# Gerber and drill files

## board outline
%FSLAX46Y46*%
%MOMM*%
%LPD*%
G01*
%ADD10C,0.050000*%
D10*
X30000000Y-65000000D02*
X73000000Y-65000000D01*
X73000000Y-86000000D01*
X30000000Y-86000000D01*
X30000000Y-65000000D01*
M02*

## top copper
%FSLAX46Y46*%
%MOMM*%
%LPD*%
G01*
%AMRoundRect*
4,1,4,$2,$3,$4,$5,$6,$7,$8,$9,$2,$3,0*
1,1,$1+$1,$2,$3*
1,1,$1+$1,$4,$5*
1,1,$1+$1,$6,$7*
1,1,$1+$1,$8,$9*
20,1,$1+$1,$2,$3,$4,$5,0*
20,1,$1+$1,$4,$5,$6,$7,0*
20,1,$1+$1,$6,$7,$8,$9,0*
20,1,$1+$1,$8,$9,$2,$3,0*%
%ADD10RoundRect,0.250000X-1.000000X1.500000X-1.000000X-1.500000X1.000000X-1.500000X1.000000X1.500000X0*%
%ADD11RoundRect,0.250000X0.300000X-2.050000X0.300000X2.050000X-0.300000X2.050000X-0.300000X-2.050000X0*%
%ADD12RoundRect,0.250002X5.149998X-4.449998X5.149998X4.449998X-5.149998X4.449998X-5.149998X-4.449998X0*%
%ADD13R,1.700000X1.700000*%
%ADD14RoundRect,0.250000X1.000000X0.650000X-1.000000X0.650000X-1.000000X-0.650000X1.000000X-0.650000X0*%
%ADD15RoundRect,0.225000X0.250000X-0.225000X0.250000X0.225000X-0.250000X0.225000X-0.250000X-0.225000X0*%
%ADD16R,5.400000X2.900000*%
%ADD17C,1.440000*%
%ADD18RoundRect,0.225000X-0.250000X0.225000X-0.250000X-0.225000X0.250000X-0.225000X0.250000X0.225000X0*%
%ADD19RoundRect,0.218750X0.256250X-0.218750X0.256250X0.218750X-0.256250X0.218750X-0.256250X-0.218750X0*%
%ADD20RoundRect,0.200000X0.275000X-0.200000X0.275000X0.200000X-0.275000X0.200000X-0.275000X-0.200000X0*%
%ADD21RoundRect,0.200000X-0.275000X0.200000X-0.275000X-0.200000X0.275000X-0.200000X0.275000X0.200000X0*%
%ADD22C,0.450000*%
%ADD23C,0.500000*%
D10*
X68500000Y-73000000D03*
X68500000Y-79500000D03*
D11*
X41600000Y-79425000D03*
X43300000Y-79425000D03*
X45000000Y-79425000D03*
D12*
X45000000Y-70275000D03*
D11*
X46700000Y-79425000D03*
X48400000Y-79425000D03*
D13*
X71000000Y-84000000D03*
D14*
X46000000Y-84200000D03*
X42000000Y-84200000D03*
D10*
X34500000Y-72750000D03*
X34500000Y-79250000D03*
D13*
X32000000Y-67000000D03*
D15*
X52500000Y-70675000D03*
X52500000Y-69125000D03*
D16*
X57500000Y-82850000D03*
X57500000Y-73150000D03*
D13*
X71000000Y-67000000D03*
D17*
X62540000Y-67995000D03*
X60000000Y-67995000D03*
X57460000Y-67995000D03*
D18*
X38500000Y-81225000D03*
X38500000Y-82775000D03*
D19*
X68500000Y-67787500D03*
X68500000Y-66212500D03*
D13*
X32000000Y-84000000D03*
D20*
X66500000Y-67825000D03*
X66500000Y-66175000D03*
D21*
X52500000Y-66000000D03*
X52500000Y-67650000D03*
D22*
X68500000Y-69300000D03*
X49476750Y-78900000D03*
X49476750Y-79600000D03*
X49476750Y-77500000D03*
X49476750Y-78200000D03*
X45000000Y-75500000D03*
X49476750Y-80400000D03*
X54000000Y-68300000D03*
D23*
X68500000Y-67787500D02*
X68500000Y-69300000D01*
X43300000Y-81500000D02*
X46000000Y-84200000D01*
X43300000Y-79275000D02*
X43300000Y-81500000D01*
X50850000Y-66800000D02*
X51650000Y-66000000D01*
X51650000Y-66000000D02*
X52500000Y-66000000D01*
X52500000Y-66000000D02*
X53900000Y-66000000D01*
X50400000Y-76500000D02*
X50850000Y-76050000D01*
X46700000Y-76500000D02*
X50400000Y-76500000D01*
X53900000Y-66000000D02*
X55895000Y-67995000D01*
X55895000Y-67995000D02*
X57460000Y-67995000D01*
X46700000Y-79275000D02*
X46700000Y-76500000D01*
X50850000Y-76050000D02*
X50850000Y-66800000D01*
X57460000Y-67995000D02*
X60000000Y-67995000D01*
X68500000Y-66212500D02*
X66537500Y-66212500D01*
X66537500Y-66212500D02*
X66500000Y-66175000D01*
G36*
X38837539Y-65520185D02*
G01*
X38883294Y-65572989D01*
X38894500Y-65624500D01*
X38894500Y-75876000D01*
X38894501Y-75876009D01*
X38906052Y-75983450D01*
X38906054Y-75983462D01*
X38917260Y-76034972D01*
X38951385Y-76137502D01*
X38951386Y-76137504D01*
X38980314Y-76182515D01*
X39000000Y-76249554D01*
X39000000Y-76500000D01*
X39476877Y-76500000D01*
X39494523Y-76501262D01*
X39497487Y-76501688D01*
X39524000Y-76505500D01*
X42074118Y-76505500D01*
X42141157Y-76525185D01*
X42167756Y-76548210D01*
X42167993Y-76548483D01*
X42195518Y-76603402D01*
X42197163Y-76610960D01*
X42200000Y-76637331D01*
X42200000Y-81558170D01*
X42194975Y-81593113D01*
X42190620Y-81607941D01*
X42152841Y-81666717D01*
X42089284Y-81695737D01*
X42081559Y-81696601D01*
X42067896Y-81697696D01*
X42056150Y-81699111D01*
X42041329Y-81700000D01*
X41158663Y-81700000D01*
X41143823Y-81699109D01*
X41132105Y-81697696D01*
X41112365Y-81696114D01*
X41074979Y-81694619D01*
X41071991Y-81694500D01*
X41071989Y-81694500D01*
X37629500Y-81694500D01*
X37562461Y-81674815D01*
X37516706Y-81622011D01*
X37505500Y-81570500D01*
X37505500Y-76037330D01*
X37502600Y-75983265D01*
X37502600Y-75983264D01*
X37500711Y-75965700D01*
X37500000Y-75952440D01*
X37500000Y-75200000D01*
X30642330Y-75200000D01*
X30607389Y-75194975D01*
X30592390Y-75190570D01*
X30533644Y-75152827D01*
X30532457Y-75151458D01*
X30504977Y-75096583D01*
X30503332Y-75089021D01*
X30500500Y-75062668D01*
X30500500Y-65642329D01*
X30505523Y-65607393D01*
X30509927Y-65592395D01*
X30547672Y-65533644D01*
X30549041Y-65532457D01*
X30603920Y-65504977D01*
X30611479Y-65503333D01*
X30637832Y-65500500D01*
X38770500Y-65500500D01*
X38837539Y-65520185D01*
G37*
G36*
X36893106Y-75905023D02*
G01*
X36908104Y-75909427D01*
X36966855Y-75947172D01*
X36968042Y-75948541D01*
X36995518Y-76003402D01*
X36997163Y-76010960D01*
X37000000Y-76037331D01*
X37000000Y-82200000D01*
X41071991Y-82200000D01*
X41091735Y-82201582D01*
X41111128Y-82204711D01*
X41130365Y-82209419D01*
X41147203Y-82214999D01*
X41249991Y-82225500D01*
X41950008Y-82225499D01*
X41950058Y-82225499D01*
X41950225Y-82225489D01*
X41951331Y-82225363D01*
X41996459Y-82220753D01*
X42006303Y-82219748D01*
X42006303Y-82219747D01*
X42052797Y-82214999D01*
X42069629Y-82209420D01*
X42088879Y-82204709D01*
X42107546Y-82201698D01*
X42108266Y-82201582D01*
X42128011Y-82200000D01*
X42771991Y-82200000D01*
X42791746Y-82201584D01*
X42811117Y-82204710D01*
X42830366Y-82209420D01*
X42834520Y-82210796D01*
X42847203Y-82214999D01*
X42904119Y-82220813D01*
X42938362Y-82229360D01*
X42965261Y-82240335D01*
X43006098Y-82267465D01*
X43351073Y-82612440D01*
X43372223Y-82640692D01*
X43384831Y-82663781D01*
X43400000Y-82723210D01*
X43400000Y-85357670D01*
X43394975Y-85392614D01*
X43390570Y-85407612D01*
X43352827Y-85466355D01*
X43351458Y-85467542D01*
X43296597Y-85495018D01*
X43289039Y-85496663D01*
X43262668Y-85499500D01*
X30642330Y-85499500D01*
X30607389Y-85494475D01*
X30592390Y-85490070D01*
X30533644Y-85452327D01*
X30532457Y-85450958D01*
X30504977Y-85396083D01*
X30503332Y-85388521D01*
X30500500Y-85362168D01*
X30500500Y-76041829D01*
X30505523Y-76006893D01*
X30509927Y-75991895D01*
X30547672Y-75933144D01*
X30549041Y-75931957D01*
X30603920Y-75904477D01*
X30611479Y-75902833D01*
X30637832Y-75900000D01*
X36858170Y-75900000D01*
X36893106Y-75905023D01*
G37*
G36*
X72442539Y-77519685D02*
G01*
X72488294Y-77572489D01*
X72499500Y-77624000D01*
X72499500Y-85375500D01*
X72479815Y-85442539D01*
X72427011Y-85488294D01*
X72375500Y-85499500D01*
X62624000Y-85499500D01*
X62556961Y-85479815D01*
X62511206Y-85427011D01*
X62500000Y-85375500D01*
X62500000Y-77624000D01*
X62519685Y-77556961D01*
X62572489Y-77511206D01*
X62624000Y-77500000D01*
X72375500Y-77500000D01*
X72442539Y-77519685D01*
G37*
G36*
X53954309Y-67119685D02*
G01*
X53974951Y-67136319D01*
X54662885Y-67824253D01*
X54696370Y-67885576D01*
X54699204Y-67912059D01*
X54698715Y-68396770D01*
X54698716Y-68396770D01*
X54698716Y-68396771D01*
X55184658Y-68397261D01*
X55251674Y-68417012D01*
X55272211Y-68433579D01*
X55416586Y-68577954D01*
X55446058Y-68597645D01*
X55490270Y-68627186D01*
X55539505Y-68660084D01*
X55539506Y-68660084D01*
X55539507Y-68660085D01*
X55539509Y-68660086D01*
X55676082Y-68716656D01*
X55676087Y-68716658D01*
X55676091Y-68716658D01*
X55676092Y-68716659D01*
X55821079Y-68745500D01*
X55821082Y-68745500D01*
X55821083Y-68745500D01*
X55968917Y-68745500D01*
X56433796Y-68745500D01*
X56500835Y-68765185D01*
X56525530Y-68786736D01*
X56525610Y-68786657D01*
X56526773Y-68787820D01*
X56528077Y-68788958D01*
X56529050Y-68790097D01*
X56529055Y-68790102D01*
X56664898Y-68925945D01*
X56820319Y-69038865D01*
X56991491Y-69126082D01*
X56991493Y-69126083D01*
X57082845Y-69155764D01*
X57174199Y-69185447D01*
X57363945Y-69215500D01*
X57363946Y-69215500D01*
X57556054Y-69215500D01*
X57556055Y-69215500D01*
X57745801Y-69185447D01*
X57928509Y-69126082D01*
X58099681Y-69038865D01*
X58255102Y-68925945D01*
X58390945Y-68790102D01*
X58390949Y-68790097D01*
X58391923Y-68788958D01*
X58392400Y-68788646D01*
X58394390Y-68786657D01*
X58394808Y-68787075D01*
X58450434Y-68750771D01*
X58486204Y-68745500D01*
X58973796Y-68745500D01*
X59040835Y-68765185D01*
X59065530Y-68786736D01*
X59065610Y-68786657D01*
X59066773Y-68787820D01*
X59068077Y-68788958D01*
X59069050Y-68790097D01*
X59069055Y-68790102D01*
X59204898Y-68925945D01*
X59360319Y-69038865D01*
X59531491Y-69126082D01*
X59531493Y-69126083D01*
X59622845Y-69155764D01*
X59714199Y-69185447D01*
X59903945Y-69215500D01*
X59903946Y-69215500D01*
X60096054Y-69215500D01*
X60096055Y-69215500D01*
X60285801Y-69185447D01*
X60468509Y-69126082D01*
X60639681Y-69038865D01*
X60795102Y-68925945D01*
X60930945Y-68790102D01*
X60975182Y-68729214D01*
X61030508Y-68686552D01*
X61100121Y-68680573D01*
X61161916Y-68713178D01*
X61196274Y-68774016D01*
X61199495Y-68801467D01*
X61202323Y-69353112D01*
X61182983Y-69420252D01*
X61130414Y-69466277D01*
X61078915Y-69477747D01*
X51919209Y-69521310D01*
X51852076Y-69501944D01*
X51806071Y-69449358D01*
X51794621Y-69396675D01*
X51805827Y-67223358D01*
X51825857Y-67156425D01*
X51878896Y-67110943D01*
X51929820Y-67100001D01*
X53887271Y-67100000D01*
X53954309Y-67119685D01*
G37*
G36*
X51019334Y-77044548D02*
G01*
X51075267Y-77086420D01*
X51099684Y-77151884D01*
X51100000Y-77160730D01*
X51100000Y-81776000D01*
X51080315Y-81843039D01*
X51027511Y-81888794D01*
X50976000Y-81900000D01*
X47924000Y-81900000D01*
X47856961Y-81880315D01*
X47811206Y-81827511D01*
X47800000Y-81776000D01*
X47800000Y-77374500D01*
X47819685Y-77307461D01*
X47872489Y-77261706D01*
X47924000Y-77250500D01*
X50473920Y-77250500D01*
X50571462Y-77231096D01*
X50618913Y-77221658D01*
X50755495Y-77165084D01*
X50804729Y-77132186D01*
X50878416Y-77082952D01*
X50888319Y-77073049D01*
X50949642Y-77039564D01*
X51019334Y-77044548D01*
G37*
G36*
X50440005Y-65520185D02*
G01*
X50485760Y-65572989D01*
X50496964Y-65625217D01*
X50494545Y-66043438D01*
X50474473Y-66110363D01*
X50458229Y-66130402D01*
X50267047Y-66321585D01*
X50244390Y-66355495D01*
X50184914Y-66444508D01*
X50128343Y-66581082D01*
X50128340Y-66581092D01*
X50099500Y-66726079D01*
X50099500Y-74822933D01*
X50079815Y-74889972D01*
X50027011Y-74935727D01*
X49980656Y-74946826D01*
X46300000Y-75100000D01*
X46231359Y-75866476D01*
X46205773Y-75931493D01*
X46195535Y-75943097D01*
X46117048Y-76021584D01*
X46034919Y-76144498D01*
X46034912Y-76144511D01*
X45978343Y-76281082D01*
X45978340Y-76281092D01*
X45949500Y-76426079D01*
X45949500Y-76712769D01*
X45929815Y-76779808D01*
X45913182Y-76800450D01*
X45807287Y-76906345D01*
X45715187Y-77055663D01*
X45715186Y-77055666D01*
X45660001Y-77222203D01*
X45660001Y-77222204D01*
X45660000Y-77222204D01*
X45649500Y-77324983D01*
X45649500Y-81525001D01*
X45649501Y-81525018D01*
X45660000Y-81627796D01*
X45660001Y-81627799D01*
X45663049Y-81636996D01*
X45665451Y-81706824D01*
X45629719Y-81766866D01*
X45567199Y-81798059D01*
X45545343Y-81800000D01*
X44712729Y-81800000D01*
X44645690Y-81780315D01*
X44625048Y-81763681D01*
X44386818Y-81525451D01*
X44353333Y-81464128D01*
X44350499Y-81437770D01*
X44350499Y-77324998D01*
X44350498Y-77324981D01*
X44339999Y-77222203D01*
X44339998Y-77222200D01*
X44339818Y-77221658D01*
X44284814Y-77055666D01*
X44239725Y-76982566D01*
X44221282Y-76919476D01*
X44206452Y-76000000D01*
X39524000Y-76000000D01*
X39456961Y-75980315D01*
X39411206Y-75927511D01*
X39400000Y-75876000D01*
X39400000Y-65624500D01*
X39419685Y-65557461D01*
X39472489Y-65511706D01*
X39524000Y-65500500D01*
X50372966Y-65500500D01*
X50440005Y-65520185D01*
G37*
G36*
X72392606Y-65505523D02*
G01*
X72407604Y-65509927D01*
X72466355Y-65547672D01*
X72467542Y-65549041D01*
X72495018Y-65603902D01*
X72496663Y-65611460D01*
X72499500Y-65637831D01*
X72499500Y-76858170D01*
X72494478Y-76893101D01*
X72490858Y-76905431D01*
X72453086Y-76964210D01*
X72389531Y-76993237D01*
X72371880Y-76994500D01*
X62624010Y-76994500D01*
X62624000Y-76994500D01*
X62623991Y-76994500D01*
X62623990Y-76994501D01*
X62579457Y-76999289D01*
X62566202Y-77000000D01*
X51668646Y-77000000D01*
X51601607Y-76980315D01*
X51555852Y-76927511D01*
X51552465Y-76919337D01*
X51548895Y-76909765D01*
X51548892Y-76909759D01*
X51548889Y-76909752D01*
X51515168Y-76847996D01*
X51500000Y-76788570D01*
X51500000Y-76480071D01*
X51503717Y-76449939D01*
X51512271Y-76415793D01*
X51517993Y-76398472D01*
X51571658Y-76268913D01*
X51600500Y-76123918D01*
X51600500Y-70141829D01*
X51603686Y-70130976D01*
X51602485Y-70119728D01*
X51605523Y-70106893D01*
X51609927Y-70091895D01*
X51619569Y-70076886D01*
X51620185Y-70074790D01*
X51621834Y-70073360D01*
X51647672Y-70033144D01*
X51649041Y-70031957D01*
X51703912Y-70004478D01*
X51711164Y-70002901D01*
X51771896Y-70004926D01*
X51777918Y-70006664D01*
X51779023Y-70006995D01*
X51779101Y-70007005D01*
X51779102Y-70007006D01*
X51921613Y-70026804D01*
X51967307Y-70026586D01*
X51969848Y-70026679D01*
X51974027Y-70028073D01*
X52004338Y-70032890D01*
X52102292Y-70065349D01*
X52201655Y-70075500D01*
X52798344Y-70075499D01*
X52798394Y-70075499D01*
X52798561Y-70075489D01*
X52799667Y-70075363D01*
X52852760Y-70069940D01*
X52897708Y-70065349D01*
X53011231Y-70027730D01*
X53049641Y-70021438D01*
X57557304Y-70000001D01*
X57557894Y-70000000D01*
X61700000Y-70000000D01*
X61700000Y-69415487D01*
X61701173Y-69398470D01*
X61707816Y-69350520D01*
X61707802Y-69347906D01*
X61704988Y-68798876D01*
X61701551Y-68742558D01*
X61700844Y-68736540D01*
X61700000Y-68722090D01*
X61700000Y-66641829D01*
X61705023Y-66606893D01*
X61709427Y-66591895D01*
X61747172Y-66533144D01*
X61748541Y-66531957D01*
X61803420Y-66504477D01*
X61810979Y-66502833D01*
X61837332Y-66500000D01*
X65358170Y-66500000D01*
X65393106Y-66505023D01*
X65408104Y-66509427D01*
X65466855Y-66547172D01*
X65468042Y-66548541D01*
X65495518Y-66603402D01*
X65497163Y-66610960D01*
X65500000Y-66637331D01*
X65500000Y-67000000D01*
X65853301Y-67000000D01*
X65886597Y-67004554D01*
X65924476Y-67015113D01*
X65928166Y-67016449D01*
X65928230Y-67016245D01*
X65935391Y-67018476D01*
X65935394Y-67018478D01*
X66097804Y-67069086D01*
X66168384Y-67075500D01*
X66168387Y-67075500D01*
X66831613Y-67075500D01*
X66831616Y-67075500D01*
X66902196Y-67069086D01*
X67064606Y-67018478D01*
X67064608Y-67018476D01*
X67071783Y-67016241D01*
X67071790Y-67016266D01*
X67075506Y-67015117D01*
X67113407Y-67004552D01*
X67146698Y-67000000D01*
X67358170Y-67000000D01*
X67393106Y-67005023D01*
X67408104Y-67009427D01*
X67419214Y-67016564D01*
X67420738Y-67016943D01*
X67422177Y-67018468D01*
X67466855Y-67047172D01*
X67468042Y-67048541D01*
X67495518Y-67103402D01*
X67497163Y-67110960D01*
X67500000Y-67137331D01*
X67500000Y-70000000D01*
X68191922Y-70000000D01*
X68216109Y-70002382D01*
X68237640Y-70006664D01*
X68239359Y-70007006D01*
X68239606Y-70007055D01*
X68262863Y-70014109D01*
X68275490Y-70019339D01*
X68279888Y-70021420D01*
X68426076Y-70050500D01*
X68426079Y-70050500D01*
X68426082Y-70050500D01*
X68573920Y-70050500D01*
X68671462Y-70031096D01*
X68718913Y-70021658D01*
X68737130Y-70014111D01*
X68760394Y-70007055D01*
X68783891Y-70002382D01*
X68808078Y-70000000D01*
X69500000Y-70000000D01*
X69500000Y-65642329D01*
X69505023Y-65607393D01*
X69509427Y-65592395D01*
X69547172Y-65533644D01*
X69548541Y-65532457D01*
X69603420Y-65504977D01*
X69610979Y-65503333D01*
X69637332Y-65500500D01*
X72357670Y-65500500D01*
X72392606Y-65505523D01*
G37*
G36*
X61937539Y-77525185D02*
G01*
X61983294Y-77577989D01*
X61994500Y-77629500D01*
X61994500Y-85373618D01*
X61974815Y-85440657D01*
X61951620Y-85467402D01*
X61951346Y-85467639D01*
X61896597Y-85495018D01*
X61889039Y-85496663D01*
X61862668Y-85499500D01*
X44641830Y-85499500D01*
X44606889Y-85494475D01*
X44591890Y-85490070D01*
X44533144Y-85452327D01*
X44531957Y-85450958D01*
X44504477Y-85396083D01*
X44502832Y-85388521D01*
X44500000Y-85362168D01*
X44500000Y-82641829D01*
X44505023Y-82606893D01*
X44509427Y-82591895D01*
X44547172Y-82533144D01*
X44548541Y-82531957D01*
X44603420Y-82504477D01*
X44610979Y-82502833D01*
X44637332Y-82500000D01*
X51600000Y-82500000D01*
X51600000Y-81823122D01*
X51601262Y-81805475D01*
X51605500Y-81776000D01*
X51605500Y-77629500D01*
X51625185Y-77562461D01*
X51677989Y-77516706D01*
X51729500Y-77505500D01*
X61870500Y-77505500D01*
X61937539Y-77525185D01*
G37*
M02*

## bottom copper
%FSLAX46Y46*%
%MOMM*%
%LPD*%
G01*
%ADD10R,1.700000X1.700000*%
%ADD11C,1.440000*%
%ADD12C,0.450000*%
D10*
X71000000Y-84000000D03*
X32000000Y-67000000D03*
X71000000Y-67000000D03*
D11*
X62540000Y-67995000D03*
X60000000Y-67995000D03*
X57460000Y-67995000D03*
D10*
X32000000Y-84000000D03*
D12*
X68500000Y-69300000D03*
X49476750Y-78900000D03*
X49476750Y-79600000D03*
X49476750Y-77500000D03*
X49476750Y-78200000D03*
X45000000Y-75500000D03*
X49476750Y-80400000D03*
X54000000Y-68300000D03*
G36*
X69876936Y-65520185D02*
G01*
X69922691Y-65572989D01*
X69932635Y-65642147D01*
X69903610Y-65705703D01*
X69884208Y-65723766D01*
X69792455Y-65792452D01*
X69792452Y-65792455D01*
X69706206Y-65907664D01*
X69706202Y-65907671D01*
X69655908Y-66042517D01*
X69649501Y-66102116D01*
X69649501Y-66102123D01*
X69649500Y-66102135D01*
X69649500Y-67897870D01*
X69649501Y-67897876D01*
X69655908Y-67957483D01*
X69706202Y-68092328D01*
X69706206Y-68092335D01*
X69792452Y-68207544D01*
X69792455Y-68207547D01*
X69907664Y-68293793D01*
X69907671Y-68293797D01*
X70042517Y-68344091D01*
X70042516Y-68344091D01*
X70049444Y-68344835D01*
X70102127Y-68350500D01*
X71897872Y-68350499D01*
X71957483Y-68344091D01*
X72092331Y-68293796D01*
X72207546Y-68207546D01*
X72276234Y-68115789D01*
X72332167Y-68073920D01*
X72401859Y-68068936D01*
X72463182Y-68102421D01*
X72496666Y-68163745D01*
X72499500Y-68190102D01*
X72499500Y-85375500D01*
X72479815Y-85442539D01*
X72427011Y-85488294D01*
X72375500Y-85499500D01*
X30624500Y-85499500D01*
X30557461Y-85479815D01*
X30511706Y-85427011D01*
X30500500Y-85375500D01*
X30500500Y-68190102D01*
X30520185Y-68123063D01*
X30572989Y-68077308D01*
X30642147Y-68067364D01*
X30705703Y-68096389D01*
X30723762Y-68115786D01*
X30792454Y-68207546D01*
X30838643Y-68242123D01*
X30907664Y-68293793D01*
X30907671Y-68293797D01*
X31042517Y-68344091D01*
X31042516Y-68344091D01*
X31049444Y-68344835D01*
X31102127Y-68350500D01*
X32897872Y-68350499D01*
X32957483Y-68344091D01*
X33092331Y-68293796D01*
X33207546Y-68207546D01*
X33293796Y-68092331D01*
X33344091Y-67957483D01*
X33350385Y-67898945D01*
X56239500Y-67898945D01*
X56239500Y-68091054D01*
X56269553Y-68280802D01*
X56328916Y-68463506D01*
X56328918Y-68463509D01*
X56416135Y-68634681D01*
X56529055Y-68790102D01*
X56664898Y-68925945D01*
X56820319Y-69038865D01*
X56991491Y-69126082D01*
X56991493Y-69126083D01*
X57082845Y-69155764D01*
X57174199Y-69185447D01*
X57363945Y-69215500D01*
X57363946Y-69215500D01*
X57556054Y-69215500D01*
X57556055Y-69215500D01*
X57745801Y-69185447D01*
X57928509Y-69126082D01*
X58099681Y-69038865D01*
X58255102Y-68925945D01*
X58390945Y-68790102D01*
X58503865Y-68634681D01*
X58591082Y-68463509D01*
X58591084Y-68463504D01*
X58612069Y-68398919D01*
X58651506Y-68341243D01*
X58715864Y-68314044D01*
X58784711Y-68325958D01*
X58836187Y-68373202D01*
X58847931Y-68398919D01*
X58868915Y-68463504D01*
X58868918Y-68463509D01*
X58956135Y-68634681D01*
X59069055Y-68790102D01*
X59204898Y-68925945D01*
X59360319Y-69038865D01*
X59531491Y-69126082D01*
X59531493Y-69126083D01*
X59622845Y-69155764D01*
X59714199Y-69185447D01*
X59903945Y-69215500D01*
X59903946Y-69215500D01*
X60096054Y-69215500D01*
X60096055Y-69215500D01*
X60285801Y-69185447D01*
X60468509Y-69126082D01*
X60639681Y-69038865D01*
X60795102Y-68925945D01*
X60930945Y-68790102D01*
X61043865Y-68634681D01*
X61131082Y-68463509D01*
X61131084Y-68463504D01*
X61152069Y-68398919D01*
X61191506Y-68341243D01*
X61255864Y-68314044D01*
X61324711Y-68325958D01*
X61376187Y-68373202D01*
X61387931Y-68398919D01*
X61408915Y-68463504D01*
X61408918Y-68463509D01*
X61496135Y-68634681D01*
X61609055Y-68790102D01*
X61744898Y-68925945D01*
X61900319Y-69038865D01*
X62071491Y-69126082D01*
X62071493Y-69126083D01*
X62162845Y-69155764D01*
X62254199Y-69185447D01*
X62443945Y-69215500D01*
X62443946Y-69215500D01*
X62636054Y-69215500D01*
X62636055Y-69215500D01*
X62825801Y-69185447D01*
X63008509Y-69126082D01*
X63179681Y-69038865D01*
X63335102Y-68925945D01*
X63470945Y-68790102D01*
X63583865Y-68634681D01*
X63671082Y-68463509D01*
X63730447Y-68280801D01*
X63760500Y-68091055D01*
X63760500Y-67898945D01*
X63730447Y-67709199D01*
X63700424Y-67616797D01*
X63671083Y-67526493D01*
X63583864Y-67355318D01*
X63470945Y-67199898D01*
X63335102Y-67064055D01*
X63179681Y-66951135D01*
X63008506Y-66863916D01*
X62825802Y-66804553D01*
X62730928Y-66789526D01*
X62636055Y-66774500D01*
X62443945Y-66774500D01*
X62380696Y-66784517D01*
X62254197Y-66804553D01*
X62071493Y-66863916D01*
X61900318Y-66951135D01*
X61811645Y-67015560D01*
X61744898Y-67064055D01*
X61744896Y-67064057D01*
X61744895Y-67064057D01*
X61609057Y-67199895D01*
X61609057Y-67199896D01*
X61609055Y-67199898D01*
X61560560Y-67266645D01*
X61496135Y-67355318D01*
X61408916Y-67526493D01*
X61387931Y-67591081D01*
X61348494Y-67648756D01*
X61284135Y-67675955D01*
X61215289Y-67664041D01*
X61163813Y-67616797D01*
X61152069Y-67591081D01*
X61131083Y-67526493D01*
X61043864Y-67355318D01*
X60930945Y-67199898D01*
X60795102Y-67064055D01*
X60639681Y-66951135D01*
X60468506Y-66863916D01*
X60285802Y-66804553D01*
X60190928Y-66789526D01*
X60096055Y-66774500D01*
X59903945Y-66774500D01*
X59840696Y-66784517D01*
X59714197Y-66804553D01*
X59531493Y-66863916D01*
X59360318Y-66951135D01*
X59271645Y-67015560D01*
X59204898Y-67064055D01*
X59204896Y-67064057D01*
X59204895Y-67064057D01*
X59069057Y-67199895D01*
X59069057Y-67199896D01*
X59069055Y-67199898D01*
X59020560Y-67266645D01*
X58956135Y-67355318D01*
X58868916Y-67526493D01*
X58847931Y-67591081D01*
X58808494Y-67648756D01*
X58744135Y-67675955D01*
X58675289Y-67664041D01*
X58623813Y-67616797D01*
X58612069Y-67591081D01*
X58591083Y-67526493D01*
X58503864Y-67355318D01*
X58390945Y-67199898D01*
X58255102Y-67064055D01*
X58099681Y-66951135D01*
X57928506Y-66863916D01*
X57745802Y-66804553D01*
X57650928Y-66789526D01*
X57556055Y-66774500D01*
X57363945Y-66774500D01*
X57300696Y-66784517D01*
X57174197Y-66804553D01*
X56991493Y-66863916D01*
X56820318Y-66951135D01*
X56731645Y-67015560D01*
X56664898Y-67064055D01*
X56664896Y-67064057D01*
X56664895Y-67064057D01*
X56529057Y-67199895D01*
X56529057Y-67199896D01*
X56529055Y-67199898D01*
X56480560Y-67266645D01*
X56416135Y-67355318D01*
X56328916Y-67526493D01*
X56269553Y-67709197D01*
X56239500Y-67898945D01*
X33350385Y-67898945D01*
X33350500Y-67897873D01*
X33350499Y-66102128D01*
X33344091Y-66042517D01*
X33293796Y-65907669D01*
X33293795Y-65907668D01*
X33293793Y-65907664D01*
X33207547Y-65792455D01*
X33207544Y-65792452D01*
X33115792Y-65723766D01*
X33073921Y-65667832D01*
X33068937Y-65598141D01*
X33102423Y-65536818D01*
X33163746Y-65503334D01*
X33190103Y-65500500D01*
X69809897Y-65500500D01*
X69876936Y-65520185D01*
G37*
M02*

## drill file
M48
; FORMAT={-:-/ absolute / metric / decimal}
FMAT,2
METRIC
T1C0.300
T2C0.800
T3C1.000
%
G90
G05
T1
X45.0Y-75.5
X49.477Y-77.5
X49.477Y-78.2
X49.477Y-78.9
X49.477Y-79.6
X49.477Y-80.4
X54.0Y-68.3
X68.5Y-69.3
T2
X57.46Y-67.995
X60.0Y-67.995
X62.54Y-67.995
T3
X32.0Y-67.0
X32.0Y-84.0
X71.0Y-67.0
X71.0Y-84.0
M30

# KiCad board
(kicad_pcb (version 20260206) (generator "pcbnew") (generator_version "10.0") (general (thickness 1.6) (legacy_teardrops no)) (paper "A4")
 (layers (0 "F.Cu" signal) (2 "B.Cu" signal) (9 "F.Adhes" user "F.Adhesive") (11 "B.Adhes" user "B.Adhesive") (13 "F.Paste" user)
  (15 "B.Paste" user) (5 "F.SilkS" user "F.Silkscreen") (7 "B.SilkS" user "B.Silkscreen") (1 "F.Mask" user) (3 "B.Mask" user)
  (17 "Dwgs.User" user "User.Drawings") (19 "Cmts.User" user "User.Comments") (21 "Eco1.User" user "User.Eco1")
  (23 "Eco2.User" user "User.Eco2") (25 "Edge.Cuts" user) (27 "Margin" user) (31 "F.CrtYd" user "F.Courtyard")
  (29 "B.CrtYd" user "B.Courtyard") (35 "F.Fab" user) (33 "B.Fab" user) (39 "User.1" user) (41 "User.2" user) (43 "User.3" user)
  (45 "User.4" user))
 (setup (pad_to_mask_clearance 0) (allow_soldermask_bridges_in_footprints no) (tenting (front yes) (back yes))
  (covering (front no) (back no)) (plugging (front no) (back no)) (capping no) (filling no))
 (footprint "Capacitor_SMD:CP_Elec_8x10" (layer "F.Cu") (at 68.5 76.25 -90)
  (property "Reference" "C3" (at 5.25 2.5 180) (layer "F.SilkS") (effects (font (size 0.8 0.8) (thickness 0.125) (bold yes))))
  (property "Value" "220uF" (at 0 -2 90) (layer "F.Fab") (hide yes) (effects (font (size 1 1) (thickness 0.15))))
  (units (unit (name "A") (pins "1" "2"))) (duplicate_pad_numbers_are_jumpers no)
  (pad "1" smd roundrect (at -3.25 0 270) (size 3.5 2.5) (layers "F.Cu" "F.Mask" "F.Paste") (roundrect_rratio 0.1) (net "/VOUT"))
  (pad "2" smd roundrect (at 3.25 0 270) (size 3.5 2.5) (layers "F.Cu" "F.Mask" "F.Paste") (roundrect_rratio 0.1) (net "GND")))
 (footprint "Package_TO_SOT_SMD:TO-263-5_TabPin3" (layer "F.Cu") (at 45 71.775 90)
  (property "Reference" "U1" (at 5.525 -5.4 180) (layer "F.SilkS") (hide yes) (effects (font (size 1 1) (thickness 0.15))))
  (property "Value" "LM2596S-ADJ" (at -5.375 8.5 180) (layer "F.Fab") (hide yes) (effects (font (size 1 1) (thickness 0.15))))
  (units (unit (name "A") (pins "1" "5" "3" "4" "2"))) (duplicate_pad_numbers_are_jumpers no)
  (pad "" smd roundrect (at -0.925 -2.775 90) (size 4.55 5.25) (layers "F.Paste") (roundrect_rratio 0.054945))
  (pad "" smd roundrect (at -0.925 2.775 90) (size 4.55 5.25) (layers "F.Paste") (roundrect_rratio 0.054945))
  (pad "" smd roundrect (at 3.925 -2.775 90) (size 4.55 5.25) (layers "F.Paste") (roundrect_rratio 0.054945))
  (pad "" smd roundrect (at 3.925 2.775 90) (size 4.55 5.25) (layers "F.Paste") (roundrect_rratio 0.054945))
  (pad "1" smd roundrect (at -7.65 -3.4 90) (size 4.6 1.1) (layers "F.Cu" "F.Mask" "F.Paste") (roundrect_rratio 0.227273) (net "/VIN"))
  (pad "2" smd roundrect (at -7.65 -1.7 90) (size 4.6 1.1) (layers "F.Cu" "F.Mask" "F.Paste") (roundrect_rratio 0.227273) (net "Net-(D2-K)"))
  (pad "3" smd roundrect (at -7.65 0 90) (size 4.6 1.1) (layers "F.Cu" "F.Mask" "F.Paste") (roundrect_rratio 0.227273) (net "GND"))
  (pad "3" smd roundrect (at 1.5 0 90) (size 9.4 10.8) (layers "F.Cu" "F.Mask") (roundrect_rratio 0.026596) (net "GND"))
  (pad "4" smd roundrect (at -7.65 1.7 90) (size 4.6 1.1) (layers "F.Cu" "F.Mask" "F.Paste") (roundrect_rratio 0.227273) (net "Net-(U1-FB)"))
  (pad "5" smd roundrect (at -7.65 3.4 90) (size 4.6 1.1) (layers "F.Cu" "F.Mask" "F.Paste") (roundrect_rratio 0.227273) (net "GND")))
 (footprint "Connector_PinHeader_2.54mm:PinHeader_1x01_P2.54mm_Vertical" (layer "F.Cu") (at 71 84)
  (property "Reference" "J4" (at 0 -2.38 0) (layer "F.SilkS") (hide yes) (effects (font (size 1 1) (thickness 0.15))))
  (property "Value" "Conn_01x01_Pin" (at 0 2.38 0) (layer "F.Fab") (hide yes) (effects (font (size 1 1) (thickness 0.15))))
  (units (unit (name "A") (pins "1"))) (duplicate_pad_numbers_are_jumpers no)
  (pad "1" thru_hole rect (at 0 0) (size 1.7 1.7) (drill 1) (layers "*.Cu" "*.Mask") (remove_unused_layers no) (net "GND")))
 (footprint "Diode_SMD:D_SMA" (layer "F.Cu") (at 44 84.2 180)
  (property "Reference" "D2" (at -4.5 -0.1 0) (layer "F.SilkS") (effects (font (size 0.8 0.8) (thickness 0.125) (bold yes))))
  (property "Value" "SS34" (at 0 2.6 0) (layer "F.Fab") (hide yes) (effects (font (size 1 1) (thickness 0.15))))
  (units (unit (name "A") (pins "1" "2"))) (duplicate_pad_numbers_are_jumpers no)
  (pad "1" smd roundrect (at -2 0 180) (size 2.5 1.8) (layers "F.Cu" "F.Mask" "F.Paste") (roundrect_rratio 0.1388888889) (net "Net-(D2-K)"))
  (pad "2" smd roundrect (at 2 0 180) (size 2.5 1.8) (layers "F.Cu" "F.Mask" "F.Paste") (roundrect_rratio 0.1388888889) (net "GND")))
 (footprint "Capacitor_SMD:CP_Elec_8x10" (layer "F.Cu") (at 34.5 76 -90)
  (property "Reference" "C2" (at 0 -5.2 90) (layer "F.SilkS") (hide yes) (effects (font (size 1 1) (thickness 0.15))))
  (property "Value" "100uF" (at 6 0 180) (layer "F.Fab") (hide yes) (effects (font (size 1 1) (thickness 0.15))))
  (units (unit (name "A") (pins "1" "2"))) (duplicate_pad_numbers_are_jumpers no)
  (pad "1" smd roundrect (at -3.25 0 270) (size 3.5 2.5) (layers "F.Cu" "F.Mask" "F.Paste") (roundrect_rratio 0.1) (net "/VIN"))
  (pad "2" smd roundrect (at 3.25 0 270) (size 3.5 2.5) (layers "F.Cu" "F.Mask" "F.Paste") (roundrect_rratio 0.1) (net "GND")))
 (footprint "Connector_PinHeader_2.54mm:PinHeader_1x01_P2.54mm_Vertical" (layer "F.Cu") (at 32 67)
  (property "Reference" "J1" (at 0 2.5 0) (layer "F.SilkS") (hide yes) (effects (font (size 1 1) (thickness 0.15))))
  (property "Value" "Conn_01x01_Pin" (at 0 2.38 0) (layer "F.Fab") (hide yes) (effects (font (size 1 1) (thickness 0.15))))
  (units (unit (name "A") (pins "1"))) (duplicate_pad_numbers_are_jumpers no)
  (pad "1" thru_hole rect (at 0 0) (size 1.7 1.7) (drill 1) (layers "*.Cu" "*.Mask") (remove_unused_layers no) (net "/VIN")))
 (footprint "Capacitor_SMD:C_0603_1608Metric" (layer "F.Cu") (at 52.5 69.9 90)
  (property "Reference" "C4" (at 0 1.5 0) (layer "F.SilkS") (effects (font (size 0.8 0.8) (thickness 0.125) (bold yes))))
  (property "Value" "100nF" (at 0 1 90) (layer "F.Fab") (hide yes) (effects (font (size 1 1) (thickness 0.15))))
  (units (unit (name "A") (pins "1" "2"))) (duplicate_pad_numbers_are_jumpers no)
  (pad "1" smd roundrect (at -0.775 0 90) (size 0.9 0.95) (layers "F.Cu" "F.Mask" "F.Paste") (roundrect_rratio 0.25) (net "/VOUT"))
  (pad "2" smd roundrect (at 0.775 0 90) (size 0.9 0.95) (layers "F.Cu" "F.Mask" "F.Paste") (roundrect_rratio 0.25) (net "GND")))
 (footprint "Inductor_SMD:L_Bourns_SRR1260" (layer "F.Cu") (at 57.5 78 90)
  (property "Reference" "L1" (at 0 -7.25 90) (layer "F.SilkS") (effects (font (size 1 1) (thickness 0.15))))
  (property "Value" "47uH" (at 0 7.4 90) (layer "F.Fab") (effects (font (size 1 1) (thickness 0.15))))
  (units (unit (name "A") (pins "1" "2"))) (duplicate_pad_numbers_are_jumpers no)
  (pad "1" smd rect (at -4.85 0 90) (size 2.9 5.4) (layers "F.Cu" "F.Mask" "F.Paste") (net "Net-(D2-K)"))
  (pad "2" smd rect (at 4.85 0 90) (size 2.9 5.4) (layers "F.Cu" "F.Mask" "F.Paste") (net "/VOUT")))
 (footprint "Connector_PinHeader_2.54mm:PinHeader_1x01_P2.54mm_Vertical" (layer "F.Cu") (at 71 67)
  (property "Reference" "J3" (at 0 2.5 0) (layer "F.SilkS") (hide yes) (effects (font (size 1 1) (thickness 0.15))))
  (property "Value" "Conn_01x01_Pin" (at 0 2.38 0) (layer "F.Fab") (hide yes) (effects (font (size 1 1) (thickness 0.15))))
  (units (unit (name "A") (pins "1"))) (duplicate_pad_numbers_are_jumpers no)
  (pad "1" thru_hole rect (at 0 0) (size 1.7 1.7) (drill 1) (layers "*.Cu" "*.Mask") (remove_unused_layers no) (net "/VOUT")))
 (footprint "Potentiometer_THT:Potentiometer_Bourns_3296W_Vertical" (layer "F.Cu") (at 62.54 67.995)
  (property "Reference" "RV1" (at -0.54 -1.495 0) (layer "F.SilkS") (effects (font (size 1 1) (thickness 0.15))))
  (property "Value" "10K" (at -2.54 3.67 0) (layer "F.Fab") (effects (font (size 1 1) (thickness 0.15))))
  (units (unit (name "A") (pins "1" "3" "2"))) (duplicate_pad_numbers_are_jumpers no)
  (pad "1" thru_hole circle (at 0 0) (size 1.44 1.44) (drill 0.8) (layers "*.Cu" "*.Mask") (remove_unused_layers no) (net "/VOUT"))
  (pad "2" thru_hole circle (at -2.54 0) (size 1.44 1.44) (drill 0.8) (layers "*.Cu" "*.Mask") (remove_unused_layers no) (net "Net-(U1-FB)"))
  (pad "3" thru_hole circle (at -5.08 0) (size 1.44 1.44) (drill 0.8) (layers "*.Cu" "*.Mask") (remove_unused_layers no) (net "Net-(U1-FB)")))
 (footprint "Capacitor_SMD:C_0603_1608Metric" (layer "F.Cu") (at 38.5 82 -90)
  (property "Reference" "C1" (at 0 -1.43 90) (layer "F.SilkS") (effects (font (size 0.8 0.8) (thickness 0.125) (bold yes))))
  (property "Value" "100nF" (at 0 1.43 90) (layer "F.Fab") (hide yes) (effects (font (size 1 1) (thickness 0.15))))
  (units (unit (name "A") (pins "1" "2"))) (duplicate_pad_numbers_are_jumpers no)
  (pad "1" smd roundrect (at -0.775 0 270) (size 0.9 0.95) (layers "F.Cu" "F.Mask" "F.Paste") (roundrect_rratio 0.25) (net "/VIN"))
  (pad "2" smd roundrect (at 0.775 0 270) (size 0.9 0.95) (layers "F.Cu" "F.Mask" "F.Paste") (roundrect_rratio 0.25) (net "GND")))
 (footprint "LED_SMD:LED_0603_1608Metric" (layer "F.Cu") (at 68.5 67 90)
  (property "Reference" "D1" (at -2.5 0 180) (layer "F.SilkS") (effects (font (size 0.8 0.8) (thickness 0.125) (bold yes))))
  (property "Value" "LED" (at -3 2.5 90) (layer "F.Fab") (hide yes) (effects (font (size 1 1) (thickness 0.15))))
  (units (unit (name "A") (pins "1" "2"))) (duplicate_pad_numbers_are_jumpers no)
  (pad "1" smd roundrect (at -0.7875 0 90) (size 0.875 0.95) (layers "F.Cu" "F.Mask" "F.Paste") (roundrect_rratio 0.25) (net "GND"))
  (pad "2" smd roundrect (at 0.7875 0 90) (size 0.875 0.95) (layers "F.Cu" "F.Mask" "F.Paste") (roundrect_rratio 0.25) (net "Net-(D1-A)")))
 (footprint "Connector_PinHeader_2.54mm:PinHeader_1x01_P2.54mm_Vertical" (layer "F.Cu") (at 32 84)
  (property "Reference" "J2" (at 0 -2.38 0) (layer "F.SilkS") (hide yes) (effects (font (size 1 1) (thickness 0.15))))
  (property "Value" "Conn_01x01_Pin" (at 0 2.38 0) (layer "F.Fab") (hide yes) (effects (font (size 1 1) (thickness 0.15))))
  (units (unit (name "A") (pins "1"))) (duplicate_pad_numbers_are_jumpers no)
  (pad "1" thru_hole rect (at 0 0) (size 1.7 1.7) (drill 1) (layers "*.Cu" "*.Mask") (remove_unused_layers no) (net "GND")))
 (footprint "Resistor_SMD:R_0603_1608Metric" (layer "F.Cu") (at 66.5 67 90)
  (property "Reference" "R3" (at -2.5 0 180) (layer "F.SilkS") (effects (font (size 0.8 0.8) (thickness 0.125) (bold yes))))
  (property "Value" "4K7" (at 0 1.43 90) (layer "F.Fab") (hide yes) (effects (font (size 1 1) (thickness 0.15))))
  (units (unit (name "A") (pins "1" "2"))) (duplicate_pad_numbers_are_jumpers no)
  (pad "1" smd roundrect (at -0.825 0 90) (size 0.8 0.95) (layers "F.Cu" "F.Mask" "F.Paste") (roundrect_rratio 0.25) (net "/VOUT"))
  (pad "2" smd roundrect (at 0.825 0 90) (size 0.8 0.95) (layers "F.Cu" "F.Mask" "F.Paste") (roundrect_rratio 0.25) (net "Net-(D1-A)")))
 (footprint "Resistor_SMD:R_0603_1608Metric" (layer "F.Cu") (at 52.5 66.825 -90)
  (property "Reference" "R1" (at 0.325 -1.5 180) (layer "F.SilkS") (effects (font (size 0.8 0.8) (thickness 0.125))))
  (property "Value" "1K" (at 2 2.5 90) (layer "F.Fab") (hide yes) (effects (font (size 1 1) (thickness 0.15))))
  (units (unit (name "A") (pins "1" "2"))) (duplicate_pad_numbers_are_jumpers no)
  (pad "1" smd roundrect (at -0.825 0 270) (size 0.8 0.95) (layers "F.Cu" "F.Mask" "F.Paste") (roundrect_rratio 0.25) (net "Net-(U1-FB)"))
  (pad "2" smd roundrect (at 0.825 0 270) (size 0.8 0.95) (layers "F.Cu" "F.Mask" "F.Paste") (roundrect_rratio 0.25) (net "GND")))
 (gr_rect (start 30 65) (end 73 86) (stroke (width 0.05) (type default)) (fill no) (layer "Edge.Cuts"))
 (segment (start 68.5 67.7875) (end 68.5 69.3) (width 0.5) (layer "F.Cu") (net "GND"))
 (via (at 68.5 69.3) (size 0.45) (drill 0.3) (layers "F.Cu" "B.Cu") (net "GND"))
 (via (at 49.47675 78.9) (size 0.45) (drill 0.3) (layers "F.Cu" "B.Cu") (free yes) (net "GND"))
 (via (at 49.47675 79.6) (size 0.45) (drill 0.3) (layers "F.Cu" "B.Cu") (free yes) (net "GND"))
 (via (at 49.47675 77.5) (size 0.45) (drill 0.3) (layers "F.Cu" "B.Cu") (free yes) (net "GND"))
 (via (at 49.47675 78.2) (size 0.45) (drill 0.3) (layers "F.Cu" "B.Cu") (free yes) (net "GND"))
 (via (at 45 75.5) (size 0.45) (drill 0.3) (layers "F.Cu" "B.Cu") (free yes) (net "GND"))
 (via (at 49.47675 80.4) (size 0.45) (drill 0.3) (layers "F.Cu" "B.Cu") (free yes) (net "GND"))
 (via (at 54 68.3) (size 0.45) (drill 0.3) (layers "F.Cu" "B.Cu") (free yes) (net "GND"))
 (segment (start 43.3 81.5) (end 46 84.2) (width 0.5) (layer "F.Cu") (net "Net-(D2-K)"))
 (segment (start 43.3 79.275) (end 43.3 81.5) (width 0.5) (layer "F.Cu") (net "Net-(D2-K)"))
 (segment (start 50.85 66.8) (end 51.65 66) (width 0.5) (layer "F.Cu") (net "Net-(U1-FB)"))
 (segment (start 51.65 66) (end 52.5 66) (width 0.5) (layer "F.Cu") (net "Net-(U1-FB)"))
 (segment (start 52.5 66) (end 53.9 66) (width 0.5) (layer "F.Cu") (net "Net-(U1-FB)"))
 (segment (start 50.4 76.5) (end 50.85 76.05) (width 0.5) (layer "F.Cu") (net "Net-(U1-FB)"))
 (segment (start 46.7 76.5) (end 50.4 76.5) (width 0.5) (layer "F.Cu") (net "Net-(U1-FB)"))
 (segment (start 53.9 66) (end 55.895 67.995) (width 0.5) (layer "F.Cu") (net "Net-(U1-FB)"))
 (segment (start 55.895 67.995) (end 57.46 67.995) (width 0.5) (layer "F.Cu") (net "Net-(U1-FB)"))
 (segment (start 46.7 79.275) (end 46.7 76.5) (width 0.5) (layer "F.Cu") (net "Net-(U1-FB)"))
 (segment (start 50.85 76.05) (end 50.85 66.8) (width 0.5) (layer "F.Cu") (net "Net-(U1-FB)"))
 (segment (start 57.46 67.995) (end 60 67.995) (width 0.5) (layer "F.Cu") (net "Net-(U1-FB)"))
 (segment (start 68.5 66.2125) (end 66.5375 66.2125) (width 0.5) (layer "F.Cu") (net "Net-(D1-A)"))
 (segment (start 66.5375 66.2125) (end 66.5 66.175) (width 0.5) (layer "F.Cu") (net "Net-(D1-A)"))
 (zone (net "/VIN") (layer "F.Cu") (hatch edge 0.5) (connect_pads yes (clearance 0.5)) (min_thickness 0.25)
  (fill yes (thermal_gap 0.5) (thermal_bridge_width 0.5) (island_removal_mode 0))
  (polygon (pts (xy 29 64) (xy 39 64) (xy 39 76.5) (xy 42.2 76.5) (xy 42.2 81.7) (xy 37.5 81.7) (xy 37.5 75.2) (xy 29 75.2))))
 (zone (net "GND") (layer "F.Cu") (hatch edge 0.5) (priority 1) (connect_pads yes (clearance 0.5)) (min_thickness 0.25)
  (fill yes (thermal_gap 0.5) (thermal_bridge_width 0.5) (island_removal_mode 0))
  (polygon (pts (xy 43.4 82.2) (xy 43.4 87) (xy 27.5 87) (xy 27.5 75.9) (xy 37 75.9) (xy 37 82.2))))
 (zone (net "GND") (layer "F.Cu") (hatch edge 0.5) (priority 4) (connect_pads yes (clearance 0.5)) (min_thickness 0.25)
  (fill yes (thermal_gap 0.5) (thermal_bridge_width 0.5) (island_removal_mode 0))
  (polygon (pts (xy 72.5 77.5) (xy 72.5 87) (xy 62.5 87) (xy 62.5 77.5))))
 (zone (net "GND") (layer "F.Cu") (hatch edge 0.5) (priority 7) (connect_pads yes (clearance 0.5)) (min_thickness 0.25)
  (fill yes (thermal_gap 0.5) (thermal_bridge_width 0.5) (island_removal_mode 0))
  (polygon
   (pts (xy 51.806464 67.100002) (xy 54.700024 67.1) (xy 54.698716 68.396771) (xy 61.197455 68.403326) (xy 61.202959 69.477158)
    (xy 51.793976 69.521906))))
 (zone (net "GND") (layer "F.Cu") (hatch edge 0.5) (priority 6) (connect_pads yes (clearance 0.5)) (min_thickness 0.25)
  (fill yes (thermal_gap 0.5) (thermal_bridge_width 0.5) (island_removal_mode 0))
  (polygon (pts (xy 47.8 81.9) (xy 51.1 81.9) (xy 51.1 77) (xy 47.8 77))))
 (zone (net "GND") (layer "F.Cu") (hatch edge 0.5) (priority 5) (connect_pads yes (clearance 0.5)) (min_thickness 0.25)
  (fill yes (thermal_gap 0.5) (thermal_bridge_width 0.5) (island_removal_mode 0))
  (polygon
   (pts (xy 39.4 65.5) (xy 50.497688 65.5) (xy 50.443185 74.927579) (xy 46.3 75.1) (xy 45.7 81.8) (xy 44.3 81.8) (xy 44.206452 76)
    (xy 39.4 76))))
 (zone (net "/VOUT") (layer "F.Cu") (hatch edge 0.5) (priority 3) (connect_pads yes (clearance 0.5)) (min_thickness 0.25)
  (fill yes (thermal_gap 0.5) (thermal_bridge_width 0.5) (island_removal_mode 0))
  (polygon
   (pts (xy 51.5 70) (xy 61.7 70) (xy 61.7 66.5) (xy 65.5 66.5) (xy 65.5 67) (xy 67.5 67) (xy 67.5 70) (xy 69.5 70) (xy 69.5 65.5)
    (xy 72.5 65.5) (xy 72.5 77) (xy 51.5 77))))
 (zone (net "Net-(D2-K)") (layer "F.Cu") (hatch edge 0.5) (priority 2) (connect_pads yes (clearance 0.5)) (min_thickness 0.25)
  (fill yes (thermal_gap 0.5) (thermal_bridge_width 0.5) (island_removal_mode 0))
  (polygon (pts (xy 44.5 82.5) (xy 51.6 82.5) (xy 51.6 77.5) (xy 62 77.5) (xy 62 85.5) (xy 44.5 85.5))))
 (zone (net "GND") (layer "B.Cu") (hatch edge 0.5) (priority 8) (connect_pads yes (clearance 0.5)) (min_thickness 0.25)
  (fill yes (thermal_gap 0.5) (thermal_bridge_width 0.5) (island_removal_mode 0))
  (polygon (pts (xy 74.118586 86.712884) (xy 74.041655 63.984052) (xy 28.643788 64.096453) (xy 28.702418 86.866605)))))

